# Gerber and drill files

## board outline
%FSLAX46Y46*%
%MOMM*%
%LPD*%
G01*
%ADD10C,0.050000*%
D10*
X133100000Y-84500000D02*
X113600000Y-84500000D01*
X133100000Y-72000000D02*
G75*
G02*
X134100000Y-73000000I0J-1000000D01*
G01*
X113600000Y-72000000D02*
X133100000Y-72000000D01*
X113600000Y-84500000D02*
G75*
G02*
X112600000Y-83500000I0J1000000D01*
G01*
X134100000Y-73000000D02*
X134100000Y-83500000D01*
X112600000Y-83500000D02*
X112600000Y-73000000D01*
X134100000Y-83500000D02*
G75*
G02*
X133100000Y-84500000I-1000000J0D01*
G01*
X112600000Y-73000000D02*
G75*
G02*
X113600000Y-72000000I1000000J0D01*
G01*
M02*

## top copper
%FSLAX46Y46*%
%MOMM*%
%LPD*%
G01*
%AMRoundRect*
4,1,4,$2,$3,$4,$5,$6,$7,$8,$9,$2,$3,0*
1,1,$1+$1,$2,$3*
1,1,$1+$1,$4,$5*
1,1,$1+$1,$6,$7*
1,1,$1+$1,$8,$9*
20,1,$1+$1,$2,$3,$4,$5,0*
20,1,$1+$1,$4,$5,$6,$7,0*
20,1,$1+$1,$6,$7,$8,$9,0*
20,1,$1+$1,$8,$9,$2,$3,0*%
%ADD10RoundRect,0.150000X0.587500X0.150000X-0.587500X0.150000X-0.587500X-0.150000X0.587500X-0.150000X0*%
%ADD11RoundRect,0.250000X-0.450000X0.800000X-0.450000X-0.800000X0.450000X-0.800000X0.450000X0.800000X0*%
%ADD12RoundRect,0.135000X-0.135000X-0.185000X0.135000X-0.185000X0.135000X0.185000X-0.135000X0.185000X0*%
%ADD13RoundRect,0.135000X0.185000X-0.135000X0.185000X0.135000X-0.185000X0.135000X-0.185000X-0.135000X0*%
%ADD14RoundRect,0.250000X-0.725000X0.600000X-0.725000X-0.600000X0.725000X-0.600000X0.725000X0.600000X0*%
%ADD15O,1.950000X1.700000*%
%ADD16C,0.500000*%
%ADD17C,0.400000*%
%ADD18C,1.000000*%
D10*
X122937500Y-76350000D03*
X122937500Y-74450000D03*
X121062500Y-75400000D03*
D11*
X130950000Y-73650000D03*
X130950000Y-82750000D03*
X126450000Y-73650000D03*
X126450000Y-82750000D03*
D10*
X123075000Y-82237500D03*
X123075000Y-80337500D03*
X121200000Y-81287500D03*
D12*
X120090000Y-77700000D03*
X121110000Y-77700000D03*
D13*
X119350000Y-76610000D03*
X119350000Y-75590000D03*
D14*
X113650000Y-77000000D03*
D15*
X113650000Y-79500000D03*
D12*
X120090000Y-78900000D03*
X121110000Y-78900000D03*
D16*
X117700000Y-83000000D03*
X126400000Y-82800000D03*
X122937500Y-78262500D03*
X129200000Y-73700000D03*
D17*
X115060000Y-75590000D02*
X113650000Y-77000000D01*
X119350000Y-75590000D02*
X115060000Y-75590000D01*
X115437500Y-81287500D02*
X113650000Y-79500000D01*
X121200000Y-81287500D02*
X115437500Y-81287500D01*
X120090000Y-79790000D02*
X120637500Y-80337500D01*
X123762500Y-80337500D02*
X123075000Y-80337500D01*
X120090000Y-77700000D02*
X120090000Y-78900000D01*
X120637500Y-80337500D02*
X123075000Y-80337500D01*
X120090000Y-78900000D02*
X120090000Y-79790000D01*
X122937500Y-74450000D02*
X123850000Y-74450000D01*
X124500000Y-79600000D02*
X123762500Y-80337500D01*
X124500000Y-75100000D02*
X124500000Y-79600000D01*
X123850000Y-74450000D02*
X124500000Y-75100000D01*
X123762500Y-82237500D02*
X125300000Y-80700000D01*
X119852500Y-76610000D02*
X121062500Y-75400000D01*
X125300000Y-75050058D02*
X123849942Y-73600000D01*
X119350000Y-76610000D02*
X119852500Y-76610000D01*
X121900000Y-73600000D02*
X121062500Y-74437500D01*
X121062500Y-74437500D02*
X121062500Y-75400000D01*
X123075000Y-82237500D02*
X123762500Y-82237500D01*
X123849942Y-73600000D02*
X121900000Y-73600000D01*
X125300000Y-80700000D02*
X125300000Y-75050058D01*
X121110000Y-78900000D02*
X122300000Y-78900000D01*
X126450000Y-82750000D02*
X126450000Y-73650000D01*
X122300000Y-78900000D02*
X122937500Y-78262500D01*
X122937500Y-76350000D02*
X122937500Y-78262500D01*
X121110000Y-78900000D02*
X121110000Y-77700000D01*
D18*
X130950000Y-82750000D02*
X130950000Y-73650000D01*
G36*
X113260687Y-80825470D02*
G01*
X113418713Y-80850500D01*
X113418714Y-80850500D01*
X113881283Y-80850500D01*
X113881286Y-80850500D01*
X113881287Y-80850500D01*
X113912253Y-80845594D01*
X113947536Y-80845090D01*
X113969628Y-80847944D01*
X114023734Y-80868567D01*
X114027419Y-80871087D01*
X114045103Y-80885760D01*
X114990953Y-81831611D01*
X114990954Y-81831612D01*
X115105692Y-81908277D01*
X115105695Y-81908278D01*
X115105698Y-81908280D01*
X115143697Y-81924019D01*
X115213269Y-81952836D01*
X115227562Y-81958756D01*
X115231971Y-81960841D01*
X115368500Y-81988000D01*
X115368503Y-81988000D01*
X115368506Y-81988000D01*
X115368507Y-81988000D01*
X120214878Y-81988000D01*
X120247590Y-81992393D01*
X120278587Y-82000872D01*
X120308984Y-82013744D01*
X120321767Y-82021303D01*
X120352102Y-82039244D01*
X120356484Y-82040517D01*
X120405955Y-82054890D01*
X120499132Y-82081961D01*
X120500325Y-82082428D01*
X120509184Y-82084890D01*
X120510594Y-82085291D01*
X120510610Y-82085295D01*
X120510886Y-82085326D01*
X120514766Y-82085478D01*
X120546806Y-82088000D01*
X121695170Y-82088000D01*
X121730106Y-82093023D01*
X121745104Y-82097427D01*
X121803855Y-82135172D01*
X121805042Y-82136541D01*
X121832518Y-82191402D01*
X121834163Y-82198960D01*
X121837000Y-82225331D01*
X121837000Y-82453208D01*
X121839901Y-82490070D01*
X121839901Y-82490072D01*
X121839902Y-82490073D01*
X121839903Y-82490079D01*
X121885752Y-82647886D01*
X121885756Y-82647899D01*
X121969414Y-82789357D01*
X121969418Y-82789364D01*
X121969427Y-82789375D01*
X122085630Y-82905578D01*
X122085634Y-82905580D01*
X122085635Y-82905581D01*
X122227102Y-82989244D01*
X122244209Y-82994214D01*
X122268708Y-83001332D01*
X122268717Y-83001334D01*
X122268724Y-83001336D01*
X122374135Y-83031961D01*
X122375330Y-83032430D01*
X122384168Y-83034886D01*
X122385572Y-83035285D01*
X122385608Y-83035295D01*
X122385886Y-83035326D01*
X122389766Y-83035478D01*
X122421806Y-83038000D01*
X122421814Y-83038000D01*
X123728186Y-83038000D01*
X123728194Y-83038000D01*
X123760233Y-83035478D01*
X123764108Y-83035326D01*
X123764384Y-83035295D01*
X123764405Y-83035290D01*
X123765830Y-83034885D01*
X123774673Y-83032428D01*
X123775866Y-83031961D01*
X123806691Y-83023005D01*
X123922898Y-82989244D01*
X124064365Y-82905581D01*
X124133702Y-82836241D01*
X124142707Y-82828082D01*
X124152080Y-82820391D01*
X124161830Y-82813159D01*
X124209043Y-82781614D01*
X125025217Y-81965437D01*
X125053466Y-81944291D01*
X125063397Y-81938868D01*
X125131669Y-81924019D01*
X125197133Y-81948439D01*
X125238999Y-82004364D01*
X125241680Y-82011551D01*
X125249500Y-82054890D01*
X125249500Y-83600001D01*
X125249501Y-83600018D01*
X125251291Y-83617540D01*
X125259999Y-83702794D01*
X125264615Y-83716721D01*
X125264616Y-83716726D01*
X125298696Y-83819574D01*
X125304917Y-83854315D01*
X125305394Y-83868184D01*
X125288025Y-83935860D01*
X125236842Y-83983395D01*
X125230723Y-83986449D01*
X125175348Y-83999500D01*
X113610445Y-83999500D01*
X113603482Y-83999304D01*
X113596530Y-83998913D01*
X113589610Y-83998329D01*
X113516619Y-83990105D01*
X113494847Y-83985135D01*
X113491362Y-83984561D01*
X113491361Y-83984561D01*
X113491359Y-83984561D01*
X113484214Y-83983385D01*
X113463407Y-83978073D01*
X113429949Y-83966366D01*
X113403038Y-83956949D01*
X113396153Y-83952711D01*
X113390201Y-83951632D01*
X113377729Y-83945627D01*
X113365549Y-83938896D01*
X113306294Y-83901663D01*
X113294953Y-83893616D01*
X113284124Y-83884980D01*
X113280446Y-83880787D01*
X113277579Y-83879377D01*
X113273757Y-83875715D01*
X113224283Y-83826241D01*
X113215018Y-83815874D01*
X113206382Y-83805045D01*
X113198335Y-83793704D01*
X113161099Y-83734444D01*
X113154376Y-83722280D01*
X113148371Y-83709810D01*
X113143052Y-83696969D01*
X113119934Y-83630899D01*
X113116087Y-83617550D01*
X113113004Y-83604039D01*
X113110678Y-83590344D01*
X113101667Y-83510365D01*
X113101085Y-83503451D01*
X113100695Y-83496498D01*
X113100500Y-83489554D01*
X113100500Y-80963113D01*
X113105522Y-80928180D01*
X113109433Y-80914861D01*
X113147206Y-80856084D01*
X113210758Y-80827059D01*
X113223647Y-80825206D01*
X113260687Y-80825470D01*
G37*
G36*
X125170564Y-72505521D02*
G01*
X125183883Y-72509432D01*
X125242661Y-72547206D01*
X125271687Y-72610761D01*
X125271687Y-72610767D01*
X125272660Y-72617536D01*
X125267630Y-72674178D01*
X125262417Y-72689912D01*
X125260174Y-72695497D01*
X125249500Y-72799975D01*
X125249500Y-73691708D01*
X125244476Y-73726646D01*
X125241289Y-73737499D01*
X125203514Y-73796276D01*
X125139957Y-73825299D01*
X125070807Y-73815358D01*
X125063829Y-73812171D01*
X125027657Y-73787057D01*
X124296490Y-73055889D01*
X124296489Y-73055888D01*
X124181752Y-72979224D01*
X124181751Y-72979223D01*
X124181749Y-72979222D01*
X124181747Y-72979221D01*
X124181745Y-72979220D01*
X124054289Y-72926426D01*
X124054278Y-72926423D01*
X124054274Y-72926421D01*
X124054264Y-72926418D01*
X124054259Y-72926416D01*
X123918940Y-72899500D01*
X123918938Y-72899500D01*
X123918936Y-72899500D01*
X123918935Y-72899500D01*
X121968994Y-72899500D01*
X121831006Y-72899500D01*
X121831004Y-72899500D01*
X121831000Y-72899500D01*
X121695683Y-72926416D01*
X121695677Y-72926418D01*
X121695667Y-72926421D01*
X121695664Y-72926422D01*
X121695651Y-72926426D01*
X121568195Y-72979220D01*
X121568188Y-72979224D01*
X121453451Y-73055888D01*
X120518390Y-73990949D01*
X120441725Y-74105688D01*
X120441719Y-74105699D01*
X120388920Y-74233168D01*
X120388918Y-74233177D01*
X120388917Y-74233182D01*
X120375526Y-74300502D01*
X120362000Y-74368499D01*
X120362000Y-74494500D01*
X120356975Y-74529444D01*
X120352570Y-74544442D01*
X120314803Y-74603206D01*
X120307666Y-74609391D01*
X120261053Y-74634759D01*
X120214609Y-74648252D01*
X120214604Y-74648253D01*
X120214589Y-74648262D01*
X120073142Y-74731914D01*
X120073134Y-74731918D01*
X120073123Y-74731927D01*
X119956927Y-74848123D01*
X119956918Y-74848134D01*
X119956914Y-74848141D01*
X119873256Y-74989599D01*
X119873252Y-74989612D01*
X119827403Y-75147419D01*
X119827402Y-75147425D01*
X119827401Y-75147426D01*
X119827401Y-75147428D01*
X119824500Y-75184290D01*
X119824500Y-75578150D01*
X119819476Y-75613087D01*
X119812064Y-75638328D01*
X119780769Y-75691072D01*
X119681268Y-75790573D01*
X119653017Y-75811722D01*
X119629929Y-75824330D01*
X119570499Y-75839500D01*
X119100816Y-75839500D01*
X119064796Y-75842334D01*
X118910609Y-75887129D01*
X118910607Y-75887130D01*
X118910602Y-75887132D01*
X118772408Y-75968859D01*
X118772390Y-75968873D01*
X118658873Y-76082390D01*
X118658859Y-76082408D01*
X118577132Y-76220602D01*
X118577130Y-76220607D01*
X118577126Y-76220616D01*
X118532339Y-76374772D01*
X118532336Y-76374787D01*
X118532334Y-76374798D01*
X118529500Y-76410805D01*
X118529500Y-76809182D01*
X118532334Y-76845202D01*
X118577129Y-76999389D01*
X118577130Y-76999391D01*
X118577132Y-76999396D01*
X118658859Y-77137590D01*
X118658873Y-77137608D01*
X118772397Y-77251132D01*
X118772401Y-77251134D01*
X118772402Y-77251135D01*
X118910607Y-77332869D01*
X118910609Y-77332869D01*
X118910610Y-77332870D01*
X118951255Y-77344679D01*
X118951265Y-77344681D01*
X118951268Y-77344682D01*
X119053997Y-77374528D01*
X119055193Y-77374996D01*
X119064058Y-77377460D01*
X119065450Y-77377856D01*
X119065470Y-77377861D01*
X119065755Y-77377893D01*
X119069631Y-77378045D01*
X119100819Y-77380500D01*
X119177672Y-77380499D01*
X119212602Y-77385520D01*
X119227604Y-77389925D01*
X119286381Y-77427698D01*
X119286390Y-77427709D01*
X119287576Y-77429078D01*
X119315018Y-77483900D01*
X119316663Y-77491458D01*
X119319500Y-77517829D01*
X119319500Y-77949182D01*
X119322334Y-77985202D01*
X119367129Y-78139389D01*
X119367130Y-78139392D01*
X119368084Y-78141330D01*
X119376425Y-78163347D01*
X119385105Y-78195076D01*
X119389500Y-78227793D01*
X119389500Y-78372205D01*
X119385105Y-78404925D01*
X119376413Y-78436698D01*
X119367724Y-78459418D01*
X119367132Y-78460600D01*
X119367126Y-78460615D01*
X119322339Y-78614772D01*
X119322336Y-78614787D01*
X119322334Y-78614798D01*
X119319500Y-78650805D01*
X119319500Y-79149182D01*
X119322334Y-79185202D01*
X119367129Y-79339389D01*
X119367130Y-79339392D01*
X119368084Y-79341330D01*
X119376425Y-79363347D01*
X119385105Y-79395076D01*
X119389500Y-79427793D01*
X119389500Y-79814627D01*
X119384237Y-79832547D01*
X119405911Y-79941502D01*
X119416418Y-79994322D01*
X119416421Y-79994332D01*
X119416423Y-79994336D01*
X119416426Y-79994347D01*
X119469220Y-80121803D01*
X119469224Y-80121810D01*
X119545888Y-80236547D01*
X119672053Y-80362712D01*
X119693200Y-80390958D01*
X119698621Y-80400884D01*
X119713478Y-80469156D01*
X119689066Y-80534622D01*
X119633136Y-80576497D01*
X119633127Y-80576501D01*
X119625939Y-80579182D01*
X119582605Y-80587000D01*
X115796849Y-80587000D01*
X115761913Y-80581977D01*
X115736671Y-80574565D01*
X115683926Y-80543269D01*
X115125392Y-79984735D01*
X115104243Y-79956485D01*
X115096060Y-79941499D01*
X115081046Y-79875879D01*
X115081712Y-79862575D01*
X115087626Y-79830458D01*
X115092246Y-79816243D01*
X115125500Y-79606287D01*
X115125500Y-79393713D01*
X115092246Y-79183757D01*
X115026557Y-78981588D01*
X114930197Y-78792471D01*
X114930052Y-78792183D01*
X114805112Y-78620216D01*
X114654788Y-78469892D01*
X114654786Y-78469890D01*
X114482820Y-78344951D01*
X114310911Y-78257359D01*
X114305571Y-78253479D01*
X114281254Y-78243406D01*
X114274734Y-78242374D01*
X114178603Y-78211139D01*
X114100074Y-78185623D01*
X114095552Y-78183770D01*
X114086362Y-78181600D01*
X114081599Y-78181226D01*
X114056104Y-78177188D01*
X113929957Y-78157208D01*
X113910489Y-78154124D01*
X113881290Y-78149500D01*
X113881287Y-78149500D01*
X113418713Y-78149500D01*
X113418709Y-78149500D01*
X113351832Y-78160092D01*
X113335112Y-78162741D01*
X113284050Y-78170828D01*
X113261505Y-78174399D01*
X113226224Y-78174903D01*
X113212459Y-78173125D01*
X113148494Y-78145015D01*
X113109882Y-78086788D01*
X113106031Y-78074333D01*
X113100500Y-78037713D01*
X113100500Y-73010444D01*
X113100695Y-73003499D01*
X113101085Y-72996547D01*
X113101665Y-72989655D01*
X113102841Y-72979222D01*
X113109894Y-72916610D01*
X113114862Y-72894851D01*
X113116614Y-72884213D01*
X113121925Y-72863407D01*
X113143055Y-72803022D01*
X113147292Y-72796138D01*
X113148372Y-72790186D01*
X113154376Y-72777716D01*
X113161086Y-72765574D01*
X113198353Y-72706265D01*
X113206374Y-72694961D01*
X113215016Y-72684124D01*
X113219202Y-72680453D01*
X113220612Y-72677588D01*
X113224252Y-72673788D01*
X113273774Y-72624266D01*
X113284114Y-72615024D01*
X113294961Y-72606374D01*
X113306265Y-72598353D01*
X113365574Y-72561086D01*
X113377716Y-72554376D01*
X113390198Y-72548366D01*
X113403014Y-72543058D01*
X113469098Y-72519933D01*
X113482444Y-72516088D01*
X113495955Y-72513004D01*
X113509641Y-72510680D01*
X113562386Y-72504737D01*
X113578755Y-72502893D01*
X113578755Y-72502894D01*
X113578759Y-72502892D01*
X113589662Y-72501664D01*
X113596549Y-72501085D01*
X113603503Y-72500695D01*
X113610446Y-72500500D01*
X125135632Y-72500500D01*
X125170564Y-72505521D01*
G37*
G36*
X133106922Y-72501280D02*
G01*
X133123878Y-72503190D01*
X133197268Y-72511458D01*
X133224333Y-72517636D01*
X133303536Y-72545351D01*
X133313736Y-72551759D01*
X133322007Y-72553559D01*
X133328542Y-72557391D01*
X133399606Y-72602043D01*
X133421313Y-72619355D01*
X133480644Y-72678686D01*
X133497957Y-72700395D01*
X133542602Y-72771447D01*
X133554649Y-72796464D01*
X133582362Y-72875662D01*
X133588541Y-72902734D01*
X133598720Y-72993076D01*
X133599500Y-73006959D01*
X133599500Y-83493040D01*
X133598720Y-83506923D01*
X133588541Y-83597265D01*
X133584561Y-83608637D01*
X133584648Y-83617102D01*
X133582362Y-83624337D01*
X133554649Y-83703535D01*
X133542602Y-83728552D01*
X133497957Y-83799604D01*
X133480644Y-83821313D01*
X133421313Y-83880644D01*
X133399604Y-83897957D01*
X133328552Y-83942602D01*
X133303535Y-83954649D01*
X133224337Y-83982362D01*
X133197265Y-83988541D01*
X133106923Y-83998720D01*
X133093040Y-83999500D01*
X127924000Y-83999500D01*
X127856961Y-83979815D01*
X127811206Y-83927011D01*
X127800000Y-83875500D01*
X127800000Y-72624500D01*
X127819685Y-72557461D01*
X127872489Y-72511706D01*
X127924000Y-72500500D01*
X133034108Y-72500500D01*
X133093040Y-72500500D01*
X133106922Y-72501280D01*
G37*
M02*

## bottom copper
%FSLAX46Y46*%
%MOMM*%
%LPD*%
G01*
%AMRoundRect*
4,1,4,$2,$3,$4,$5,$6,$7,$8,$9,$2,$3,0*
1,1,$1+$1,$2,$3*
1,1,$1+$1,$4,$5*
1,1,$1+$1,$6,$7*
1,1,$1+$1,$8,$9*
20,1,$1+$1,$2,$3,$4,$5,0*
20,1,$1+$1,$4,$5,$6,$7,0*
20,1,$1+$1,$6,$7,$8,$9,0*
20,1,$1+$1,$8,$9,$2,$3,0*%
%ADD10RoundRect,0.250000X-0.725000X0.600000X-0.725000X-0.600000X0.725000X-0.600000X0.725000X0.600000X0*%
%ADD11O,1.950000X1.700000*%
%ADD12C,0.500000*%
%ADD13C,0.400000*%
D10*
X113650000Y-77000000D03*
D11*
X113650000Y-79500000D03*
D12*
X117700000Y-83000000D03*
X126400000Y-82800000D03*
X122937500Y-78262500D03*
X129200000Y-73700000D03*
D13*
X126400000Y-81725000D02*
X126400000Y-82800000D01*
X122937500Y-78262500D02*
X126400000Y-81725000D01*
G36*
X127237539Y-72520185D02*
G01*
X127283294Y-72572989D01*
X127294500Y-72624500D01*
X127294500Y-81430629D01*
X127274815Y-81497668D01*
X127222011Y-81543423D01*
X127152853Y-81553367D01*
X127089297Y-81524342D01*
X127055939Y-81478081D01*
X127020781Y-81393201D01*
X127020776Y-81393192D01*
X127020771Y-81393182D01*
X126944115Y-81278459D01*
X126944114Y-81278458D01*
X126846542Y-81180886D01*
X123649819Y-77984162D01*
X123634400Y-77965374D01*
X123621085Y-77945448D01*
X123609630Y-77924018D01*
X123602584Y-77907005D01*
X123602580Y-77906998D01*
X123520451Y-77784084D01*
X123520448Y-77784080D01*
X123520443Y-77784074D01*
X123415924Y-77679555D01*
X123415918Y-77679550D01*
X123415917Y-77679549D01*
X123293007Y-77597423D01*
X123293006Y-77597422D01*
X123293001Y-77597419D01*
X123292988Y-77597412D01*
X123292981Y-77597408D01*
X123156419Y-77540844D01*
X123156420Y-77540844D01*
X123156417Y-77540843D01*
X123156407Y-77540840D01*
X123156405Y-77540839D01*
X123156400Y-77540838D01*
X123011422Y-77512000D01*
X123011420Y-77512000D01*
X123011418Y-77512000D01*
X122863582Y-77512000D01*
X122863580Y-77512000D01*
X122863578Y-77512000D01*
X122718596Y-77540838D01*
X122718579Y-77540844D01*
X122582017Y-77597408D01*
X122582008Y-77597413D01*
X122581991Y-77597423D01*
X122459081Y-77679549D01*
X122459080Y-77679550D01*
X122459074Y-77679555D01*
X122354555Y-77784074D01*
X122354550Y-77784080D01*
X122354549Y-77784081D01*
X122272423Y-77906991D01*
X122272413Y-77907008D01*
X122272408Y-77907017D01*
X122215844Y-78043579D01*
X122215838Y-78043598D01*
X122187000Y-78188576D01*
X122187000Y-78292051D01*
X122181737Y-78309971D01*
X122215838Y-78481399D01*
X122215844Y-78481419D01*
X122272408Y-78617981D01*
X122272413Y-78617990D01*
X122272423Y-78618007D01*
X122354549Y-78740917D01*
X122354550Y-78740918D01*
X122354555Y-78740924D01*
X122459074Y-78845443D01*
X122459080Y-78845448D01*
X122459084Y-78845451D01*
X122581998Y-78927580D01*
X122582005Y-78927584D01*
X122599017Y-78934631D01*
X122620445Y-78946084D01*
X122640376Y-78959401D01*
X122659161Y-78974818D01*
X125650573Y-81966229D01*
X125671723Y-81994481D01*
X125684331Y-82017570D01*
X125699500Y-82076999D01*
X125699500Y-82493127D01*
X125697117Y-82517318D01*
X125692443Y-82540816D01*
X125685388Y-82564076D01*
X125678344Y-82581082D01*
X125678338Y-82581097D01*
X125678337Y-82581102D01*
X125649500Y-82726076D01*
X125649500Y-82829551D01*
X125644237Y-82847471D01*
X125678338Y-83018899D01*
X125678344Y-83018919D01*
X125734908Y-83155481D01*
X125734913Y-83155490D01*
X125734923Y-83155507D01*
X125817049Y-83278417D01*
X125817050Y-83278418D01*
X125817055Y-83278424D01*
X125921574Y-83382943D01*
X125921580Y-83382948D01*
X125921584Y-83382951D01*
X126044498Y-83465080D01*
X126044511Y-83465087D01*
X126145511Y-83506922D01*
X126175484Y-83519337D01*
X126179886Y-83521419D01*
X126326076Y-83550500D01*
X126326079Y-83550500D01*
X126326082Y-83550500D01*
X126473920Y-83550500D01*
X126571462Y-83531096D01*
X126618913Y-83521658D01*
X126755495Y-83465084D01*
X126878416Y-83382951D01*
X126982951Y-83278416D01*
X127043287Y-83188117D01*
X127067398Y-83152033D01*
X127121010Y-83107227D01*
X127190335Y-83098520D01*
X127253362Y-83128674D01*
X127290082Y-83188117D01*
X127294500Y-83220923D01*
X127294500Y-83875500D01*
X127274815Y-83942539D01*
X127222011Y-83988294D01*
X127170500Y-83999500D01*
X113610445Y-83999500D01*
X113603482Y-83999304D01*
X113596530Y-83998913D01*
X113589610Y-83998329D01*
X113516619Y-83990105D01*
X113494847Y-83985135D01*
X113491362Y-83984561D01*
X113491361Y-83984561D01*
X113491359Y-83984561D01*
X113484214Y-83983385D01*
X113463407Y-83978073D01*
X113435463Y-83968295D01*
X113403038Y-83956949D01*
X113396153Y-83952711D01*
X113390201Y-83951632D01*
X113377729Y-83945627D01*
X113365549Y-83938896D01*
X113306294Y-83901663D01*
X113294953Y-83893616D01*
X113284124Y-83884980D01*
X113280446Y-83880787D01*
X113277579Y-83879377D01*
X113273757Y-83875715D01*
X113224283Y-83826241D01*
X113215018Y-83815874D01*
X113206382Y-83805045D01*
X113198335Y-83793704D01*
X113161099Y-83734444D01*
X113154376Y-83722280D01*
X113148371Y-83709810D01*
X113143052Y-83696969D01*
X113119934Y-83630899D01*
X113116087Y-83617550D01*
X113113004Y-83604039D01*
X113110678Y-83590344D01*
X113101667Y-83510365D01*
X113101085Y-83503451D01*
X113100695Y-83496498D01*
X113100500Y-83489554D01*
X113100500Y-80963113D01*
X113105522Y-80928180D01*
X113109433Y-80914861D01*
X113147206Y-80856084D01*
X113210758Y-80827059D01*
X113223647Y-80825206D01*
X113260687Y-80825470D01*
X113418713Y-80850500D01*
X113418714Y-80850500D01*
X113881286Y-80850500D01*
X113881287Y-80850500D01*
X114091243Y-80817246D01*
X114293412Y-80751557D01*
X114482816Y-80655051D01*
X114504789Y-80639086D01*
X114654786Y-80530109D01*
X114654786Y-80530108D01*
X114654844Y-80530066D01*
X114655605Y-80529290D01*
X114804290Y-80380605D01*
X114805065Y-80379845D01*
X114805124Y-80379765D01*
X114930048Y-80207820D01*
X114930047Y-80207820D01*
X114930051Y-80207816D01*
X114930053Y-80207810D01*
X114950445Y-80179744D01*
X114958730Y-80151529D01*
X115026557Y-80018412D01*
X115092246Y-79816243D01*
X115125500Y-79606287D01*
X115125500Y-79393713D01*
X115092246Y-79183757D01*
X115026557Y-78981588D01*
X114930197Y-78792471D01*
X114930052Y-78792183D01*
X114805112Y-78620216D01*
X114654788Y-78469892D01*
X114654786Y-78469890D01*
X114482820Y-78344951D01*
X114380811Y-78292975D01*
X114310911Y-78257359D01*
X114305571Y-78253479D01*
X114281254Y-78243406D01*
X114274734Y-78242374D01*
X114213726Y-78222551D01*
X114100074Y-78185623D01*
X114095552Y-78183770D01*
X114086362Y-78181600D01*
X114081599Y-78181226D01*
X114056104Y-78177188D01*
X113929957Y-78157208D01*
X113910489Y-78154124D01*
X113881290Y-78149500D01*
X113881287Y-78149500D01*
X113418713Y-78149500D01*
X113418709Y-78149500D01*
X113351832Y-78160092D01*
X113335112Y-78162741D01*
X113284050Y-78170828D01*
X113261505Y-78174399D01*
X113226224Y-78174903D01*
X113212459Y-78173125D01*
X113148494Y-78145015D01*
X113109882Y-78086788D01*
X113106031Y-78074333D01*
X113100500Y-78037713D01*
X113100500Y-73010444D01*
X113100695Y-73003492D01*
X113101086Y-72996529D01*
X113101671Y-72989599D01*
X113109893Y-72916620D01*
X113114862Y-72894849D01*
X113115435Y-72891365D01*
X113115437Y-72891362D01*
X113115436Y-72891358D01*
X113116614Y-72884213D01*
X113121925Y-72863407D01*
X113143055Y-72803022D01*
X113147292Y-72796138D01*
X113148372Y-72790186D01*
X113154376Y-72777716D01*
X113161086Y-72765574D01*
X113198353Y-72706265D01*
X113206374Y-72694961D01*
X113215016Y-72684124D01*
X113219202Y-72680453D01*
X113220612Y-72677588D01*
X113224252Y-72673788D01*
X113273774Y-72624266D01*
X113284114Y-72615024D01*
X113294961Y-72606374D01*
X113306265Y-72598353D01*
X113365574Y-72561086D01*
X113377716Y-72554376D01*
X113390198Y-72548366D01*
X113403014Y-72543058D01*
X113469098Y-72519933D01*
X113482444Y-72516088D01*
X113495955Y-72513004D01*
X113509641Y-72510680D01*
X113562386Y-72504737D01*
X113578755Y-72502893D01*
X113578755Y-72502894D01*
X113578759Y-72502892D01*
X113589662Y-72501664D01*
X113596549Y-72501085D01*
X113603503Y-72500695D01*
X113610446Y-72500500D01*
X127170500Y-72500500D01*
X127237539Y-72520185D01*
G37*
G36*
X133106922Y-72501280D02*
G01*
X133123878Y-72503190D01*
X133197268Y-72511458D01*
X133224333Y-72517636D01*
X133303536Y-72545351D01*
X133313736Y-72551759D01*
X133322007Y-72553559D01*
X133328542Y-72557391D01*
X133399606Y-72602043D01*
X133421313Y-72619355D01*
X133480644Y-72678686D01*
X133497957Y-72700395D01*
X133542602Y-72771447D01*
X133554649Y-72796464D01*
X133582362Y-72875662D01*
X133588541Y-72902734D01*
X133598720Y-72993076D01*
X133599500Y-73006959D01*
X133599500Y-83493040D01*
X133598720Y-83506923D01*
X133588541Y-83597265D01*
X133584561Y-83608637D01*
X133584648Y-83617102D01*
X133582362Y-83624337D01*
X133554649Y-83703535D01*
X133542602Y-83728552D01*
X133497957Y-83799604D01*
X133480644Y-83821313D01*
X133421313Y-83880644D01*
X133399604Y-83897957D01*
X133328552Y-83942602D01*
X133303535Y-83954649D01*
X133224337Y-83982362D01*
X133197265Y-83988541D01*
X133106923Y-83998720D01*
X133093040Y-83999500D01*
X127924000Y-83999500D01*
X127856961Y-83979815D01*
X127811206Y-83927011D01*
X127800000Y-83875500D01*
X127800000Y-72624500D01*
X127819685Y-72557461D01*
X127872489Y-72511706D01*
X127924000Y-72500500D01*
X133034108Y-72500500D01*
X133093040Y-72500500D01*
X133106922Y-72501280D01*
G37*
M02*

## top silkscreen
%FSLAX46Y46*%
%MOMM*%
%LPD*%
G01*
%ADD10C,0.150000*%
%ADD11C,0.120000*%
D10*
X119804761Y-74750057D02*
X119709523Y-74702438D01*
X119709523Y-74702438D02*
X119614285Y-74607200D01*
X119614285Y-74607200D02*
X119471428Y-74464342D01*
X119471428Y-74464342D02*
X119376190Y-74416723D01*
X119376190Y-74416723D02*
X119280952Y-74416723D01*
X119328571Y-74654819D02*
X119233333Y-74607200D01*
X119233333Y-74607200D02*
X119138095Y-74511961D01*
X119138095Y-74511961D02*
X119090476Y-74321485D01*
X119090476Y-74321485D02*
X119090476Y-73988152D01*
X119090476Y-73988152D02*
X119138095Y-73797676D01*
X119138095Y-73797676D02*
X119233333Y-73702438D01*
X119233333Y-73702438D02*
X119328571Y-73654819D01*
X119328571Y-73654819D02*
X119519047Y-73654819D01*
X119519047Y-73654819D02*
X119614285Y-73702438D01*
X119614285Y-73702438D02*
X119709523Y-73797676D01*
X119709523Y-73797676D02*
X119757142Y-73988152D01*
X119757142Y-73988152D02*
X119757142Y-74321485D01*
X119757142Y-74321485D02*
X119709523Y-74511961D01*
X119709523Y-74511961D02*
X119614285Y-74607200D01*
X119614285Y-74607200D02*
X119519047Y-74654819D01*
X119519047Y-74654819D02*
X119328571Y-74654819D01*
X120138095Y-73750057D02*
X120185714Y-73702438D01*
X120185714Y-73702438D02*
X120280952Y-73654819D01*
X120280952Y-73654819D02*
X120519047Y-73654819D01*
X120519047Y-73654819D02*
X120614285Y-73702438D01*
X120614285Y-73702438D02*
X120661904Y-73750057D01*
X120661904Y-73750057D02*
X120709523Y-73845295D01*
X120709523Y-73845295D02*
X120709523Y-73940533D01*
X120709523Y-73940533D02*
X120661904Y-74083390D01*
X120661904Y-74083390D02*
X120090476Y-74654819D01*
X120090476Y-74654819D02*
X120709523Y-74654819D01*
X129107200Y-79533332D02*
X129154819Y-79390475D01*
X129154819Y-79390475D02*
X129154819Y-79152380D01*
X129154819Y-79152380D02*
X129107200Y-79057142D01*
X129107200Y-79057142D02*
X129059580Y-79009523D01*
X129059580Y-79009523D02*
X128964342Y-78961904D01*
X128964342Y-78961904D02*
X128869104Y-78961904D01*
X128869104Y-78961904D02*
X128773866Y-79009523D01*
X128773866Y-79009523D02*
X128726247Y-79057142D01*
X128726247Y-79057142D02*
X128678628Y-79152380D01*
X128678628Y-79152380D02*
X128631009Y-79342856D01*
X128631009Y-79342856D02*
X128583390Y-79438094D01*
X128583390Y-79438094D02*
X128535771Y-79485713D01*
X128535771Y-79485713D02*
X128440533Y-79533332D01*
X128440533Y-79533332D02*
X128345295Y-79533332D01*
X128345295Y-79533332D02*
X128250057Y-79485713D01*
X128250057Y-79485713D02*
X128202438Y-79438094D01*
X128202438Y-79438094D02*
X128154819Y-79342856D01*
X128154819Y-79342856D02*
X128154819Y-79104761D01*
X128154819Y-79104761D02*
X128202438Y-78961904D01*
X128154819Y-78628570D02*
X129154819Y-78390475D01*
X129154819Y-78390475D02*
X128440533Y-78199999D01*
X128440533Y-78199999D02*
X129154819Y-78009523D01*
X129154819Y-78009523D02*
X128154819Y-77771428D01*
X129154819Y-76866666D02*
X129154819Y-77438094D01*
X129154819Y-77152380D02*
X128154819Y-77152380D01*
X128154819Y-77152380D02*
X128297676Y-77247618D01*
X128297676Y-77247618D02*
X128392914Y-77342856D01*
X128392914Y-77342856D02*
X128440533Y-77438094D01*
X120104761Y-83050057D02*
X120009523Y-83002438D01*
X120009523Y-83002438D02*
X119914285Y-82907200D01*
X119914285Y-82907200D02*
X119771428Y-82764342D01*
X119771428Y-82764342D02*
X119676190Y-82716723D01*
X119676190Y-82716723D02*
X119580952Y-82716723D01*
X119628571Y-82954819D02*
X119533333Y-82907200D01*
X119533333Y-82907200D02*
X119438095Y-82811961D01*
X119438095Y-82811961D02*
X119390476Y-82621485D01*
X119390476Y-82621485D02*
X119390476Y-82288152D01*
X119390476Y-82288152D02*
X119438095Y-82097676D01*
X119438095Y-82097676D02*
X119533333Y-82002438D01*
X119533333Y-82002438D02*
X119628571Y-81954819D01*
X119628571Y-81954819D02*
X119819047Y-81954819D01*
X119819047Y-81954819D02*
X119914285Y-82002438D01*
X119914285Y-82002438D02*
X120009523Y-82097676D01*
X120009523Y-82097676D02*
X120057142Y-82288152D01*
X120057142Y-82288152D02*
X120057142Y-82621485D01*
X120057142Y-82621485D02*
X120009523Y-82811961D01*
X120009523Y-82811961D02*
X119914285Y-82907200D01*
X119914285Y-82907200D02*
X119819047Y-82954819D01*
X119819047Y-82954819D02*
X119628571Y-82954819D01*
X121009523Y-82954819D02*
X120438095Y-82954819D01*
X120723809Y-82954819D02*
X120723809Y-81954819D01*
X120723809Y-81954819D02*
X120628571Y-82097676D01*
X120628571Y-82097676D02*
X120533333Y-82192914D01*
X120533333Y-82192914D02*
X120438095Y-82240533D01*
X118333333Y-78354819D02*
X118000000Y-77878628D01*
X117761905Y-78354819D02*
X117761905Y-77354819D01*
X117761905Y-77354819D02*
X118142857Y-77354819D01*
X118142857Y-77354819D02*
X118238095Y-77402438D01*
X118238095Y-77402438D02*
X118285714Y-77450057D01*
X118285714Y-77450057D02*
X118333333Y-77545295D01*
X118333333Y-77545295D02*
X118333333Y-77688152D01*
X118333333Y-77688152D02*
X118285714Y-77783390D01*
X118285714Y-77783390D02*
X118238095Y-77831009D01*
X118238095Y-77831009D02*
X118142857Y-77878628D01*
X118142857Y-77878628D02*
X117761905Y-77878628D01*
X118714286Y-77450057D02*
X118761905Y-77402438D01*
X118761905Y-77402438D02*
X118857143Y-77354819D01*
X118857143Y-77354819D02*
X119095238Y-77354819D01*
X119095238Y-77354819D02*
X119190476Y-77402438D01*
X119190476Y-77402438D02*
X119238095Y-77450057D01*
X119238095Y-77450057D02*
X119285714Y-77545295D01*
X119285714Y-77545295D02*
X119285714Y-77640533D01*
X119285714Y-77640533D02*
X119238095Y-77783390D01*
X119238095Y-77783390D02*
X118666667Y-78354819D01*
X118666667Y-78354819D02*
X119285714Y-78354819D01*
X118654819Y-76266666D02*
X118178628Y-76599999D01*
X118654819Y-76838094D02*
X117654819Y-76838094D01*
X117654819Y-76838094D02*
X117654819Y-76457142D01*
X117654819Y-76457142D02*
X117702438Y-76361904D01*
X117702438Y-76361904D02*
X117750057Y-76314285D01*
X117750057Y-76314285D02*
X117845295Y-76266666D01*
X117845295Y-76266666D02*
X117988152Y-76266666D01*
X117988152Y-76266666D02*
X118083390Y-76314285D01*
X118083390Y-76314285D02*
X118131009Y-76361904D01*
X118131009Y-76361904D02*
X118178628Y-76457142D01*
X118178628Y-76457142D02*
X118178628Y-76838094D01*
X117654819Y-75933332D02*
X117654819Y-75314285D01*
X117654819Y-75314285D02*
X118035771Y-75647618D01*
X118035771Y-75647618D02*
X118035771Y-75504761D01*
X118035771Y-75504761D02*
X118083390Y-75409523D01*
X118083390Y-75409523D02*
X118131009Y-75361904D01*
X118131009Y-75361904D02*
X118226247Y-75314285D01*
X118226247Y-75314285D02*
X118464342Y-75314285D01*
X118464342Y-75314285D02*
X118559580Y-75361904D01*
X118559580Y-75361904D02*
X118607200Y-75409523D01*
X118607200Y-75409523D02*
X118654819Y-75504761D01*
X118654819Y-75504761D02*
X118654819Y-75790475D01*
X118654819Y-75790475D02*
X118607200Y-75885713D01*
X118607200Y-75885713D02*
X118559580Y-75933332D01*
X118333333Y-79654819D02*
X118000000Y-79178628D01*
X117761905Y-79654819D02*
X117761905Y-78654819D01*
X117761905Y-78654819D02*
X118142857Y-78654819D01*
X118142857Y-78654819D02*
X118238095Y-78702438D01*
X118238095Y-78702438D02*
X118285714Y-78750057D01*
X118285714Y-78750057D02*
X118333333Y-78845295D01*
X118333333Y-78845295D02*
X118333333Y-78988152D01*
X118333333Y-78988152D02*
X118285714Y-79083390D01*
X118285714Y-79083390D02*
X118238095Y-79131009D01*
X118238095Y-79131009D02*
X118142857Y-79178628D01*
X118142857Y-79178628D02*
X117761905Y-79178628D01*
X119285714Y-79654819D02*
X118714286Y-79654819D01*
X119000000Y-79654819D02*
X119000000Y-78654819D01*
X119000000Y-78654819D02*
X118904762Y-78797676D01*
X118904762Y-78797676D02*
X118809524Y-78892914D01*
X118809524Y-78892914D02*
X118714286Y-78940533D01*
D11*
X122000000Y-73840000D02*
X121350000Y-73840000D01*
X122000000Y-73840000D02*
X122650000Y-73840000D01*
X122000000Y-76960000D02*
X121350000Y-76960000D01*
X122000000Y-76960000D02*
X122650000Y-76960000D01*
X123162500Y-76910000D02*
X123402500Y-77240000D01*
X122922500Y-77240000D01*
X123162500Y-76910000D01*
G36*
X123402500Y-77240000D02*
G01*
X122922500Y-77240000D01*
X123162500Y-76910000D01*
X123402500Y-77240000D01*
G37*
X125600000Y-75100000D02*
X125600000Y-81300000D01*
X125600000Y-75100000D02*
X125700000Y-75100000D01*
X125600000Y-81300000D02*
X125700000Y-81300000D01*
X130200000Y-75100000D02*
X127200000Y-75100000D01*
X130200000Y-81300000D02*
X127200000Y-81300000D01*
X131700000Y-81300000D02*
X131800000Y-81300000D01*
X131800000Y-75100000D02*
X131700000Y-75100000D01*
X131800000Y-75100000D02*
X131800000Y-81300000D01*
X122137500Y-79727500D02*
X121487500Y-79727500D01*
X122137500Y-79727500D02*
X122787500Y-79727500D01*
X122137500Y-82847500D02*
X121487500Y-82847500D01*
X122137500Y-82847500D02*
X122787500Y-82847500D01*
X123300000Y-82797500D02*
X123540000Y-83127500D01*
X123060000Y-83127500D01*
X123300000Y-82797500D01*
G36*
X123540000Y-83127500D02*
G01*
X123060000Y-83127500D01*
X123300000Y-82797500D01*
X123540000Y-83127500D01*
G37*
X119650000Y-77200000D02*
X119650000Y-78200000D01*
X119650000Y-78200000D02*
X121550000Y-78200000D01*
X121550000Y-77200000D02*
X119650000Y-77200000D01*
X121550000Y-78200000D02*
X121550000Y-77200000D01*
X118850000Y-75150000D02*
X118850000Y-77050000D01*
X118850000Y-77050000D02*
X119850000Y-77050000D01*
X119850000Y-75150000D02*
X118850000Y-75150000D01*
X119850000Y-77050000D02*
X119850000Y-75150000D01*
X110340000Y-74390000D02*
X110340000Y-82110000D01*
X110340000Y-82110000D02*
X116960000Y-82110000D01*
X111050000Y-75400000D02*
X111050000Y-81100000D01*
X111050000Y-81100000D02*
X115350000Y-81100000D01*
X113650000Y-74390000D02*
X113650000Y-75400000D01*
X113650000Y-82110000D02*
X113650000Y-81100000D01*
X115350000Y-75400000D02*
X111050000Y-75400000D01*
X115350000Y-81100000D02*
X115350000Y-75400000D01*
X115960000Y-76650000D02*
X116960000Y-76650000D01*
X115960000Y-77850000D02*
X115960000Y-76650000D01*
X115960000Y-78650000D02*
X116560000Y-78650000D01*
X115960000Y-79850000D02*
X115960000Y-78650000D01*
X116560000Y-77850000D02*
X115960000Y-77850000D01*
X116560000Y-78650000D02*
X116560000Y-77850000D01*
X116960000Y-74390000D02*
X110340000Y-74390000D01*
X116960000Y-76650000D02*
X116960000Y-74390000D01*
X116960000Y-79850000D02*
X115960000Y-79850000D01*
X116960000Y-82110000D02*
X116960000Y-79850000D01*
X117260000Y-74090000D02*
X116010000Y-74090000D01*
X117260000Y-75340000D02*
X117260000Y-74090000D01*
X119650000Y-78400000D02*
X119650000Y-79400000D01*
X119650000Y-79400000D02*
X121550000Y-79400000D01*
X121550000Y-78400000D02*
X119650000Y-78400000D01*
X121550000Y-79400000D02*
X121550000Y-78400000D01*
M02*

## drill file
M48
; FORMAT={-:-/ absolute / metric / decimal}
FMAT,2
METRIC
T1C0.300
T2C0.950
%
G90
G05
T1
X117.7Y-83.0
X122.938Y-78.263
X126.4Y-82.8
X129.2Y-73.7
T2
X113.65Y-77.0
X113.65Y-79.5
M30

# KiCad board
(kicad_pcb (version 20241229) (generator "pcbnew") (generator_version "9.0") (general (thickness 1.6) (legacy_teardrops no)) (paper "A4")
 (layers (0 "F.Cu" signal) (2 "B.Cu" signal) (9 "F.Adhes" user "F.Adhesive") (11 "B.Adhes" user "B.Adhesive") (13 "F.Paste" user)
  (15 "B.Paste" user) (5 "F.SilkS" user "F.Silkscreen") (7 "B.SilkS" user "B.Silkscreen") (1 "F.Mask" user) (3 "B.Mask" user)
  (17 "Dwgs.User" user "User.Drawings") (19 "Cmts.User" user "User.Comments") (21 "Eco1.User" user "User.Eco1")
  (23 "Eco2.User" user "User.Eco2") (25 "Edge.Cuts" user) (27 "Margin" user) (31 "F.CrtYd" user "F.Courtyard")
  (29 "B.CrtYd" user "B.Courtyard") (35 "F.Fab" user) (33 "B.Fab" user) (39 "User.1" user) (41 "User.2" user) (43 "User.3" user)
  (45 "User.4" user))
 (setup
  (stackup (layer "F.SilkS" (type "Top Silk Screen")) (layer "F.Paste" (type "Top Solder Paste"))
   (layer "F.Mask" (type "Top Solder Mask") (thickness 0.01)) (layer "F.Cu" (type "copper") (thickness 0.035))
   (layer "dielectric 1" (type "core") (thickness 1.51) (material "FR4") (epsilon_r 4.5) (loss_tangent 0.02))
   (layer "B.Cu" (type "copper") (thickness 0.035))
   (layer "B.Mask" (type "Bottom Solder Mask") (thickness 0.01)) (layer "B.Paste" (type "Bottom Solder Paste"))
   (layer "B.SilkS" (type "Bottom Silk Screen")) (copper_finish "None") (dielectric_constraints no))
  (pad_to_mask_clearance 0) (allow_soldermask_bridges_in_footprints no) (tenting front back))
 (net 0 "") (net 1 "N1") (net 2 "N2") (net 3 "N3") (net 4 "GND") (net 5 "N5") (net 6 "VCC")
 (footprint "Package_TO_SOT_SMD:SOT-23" (layer "F.Cu") (at 122 75.4 180)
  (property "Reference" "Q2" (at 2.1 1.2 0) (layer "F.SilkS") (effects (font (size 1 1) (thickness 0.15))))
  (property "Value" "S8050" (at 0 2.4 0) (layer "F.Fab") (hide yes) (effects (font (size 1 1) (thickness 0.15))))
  (fp_line (start 0 1.56) (end 0.65 1.56) (stroke (width 0.12) (type solid)) (layer "F.SilkS"))
  (fp_line (start 0 1.56) (end -0.65 1.56) (stroke (width 0.12) (type solid)) (layer "F.SilkS"))
  (fp_line (start 0 -1.56) (end 0.65 -1.56) (stroke (width 0.12) (type solid)) (layer "F.SilkS"))
  (fp_line (start 0 -1.56) (end -0.65 -1.56) (stroke (width 0.12) (type solid)) (layer "F.SilkS"))
  (fp_poly (pts (xy -1.1625 -1.51) (xy -1.4025 -1.84) (xy -0.9225 -1.84)) (stroke (width 0.12) (type solid)) (fill yes) (layer "F.SilkS"))
  (pad "1" smd roundrect (at -0.9375 -0.95 180) (size 1.475 0.6) (layers "F.Cu" "F.Mask" "F.Paste") (roundrect_rratio 0.25) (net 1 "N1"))
  (pad "2" smd roundrect (at -0.9375 0.95 180) (size 1.475 0.6) (layers "F.Cu" "F.Mask" "F.Paste") (roundrect_rratio 0.25) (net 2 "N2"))
  (pad "3" smd roundrect (at 0.9375 0 180) (size 1.475 0.6) (layers "F.Cu" "F.Mask" "F.Paste") (roundrect_rratio 0.25) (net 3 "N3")))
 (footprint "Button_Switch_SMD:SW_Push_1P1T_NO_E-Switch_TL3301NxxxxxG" (layer "F.Cu") (at 128.7 78.2 -90)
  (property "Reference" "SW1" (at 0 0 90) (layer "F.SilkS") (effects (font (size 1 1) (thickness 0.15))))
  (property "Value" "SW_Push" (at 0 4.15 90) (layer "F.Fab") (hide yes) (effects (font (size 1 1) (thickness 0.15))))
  (fp_line (start -3.1 3.1) (end 3.1 3.1) (stroke (width 0.12) (type solid)) (layer "F.SilkS"))
  (fp_line (start -3.1 3.1) (end -3.1 3) (stroke (width 0.12) (type solid)) (layer "F.SilkS"))
  (fp_line (start 3.1 3.1) (end 3.1 3) (stroke (width 0.12) (type solid)) (layer "F.SilkS"))
  (fp_line (start -3.1 -1.5) (end -3.1 1.5) (stroke (width 0.12) (type solid)) (layer "F.SilkS"))
  (fp_line (start 3.1 -1.5) (end 3.1 1.5) (stroke (width 0.12) (type solid)) (layer "F.SilkS"))
  (fp_line (start 3.1 -3) (end 3.1 -3.1) (stroke (width 0.12) (type solid)) (layer "F.SilkS"))
  (fp_line (start -3.1 -3.1) (end -3.1 -3) (stroke (width 0.12) (type solid)) (layer "F.SilkS"))
  (fp_line (start -3.1 -3.1) (end 3.1 -3.1) (stroke (width 0.12) (type solid)) (layer "F.SilkS"))
  (pad "1" smd roundrect (at -4.55 -2.25 270) (size 2.1 1.4) (layers "F.Cu" "F.Mask" "F.Paste") (roundrect_rratio 0.1785714286)
   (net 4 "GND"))
  (pad "1" smd roundrect (at 4.55 -2.25 270) (size 2.1 1.4) (layers "F.Cu" "F.Mask" "F.Paste") (roundrect_rratio 0.1785714286) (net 4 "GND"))
  (pad "2" smd roundrect (at -4.55 2.25 270) (size 2.1 1.4) (layers "F.Cu" "F.Mask" "F.Paste") (roundrect_rratio 0.1785714286) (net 1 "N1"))
  (pad "2" smd roundrect (at 4.55 2.25 270) (size 2.1 1.4) (layers "F.Cu" "F.Mask" "F.Paste") (roundrect_rratio 0.1785714286) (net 1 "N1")))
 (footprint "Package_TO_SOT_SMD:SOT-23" (layer "F.Cu") (at 122.1375 81.2875 180)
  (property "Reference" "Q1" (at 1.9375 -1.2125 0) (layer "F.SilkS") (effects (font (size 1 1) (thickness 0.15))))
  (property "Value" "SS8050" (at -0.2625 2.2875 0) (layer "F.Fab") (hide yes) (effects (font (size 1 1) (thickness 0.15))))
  (fp_line (start 0 1.56) (end 0.65 1.56) (stroke (width 0.12) (type solid)) (layer "F.SilkS"))
  (fp_line (start 0 1.56) (end -0.65 1.56) (stroke (width 0.12) (type solid)) (layer "F.SilkS"))
  (fp_line (start 0 -1.56) (end 0.65 -1.56) (stroke (width 0.12) (type solid)) (layer "F.SilkS"))
  (fp_line (start 0 -1.56) (end -0.65 -1.56) (stroke (width 0.12) (type solid)) (layer "F.SilkS"))
  (fp_poly (pts (xy -1.1625 -1.51) (xy -1.4025 -1.84) (xy -0.9225 -1.84)) (stroke (width 0.12) (type solid)) (fill yes) (layer "F.SilkS"))
  (pad "1" smd roundrect (at -0.9375 -0.95 180) (size 1.475 0.6) (layers "F.Cu" "F.Mask" "F.Paste") (roundrect_rratio 0.25) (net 3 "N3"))
  (pad "2" smd roundrect (at -0.9375 0.95 180) (size 1.475 0.6) (layers "F.Cu" "F.Mask" "F.Paste") (roundrect_rratio 0.25) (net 2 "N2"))
  (pad "3" smd roundrect (at 0.9375 0 180) (size 1.475 0.6) (layers "F.Cu" "F.Mask" "F.Paste") (roundrect_rratio 0.25) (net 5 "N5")))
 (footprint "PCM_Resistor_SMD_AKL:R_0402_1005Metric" (layer "F.Cu") (at 120.6 77.7)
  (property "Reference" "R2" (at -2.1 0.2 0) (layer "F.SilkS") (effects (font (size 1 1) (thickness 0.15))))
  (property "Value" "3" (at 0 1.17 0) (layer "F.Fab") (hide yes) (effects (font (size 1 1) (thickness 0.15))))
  (fp_line (start -0.95 -0.5) (end -0.95 0.5) (stroke (width 0.12) (type solid)) (layer "F.SilkS"))
  (fp_line (start -0.95 0.5) (end 0.95 0.5) (stroke (width 0.12) (type solid)) (layer "F.SilkS"))
  (fp_line (start 0.95 -0.5) (end -0.95 -0.5) (stroke (width 0.12) (type solid)) (layer "F.SilkS"))
  (fp_line (start 0.95 0.5) (end 0.95 -0.5) (stroke (width 0.12) (type solid)) (layer "F.SilkS"))
  (pad "1" smd roundrect (at -0.51 0) (size 0.54 0.64) (layers "F.Cu" "F.Mask" "F.Paste") (roundrect_rratio 0.25) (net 2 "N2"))
  (pad "2" smd roundrect (at 0.51 0) (size 0.54 0.64) (layers "F.Cu" "F.Mask" "F.Paste") (roundrect_rratio 0.25) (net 1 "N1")))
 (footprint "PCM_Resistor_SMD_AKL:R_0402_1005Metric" (layer "F.Cu") (at 119.35 76.1 90)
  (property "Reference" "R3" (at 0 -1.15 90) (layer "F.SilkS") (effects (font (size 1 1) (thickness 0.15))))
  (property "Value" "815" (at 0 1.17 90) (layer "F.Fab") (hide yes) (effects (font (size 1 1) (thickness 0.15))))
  (fp_line (start 0.95 -0.5) (end -0.95 -0.5) (stroke (width 0.12) (type solid)) (layer "F.SilkS"))
  (fp_line (start -0.95 -0.5) (end -0.95 0.5) (stroke (width 0.12) (type solid)) (layer "F.SilkS"))
  (fp_line (start 0.95 0.5) (end 0.95 -0.5) (stroke (width 0.12) (type solid)) (layer "F.SilkS"))
  (fp_line (start -0.95 0.5) (end 0.95 0.5) (stroke (width 0.12) (type solid)) (layer "F.SilkS"))
  (pad "1" smd roundrect (at -0.51 0 90) (size 0.54 0.64) (layers "F.Cu" "F.Mask" "F.Paste") (roundrect_rratio 0.25) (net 3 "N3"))
  (pad "2" smd roundrect (at 0.51 0 90) (size 0.54 0.64) (layers "F.Cu" "F.Mask" "F.Paste") (roundrect_rratio 0.25) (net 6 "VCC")))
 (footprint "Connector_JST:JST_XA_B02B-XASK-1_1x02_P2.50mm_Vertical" (layer "F.Cu") (at 113.65 77 -90)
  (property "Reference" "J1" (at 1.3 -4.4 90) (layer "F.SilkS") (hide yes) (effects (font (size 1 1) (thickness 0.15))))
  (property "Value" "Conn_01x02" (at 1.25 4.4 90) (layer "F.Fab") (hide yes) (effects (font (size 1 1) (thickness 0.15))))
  (fp_line (start -2.61 3.31) (end 5.11 3.31) (stroke (width 0.12) (type solid)) (layer "F.SilkS"))
  (fp_line (start 5.11 3.31) (end 5.11 -3.31) (stroke (width 0.12) (type solid)) (layer "F.SilkS"))
  (fp_line (start -1.6 2.6) (end 4.1 2.6) (stroke (width 0.12) (type solid)) (layer "F.SilkS"))
  (fp_line (start 4.1 2.6) (end 4.1 -1.7) (stroke (width 0.12) (type solid)) (layer "F.SilkS"))
  (fp_line (start -2.61 0) (end -1.6 0) (stroke (width 0.12) (type solid)) (layer "F.SilkS"))
  (fp_line (start 5.11 0) (end 4.1 0) (stroke (width 0.12) (type solid)) (layer "F.SilkS"))
  (fp_line (start -1.6 -1.7) (end -1.6 2.6) (stroke (width 0.12) (type solid)) (layer "F.SilkS"))
  (fp_line (start 4.1 -1.7) (end -1.6 -1.7) (stroke (width 0.12) (type solid)) (layer "F.SilkS"))
  (fp_line (start -0.35 -2.31) (end -0.35 -3.31) (stroke (width 0.12) (type solid)) (layer "F.SilkS"))
  (fp_line (start 0.85 -2.31) (end -0.35 -2.31) (stroke (width 0.12) (type solid)) (layer "F.SilkS"))
  (fp_line (start 1.65 -2.31) (end 1.65 -2.91) (stroke (width 0.12) (type solid)) (layer "F.SilkS"))
  (fp_line (start 2.85 -2.31) (end 1.65 -2.31) (stroke (width 0.12) (type solid)) (layer "F.SilkS"))
  (fp_line (start 0.85 -2.91) (end 0.85 -2.31) (stroke (width 0.12) (type solid)) (layer "F.SilkS"))
  (fp_line (start 1.65 -2.91) (end 0.85 -2.91) (stroke (width 0.12) (type solid)) (layer "F.SilkS"))
  (fp_line (start -2.61 -3.31) (end -2.61 3.31) (stroke (width 0.12) (type solid)) (layer "F.SilkS"))
  (fp_line (start -0.35 -3.31) (end -2.61 -3.31) (stroke (width 0.12) (type solid)) (layer "F.SilkS"))
  (fp_line (start 2.85 -3.31) (end 2.85 -2.31) (stroke (width 0.12) (type solid)) (layer "F.SilkS"))
  (fp_line (start 5.11 -3.31) (end 2.85 -3.31) (stroke (width 0.12) (type solid)) (layer "F.SilkS"))
  (fp_line (start -2.91 -3.61) (end -2.91 -2.36) (stroke (width 0.12) (type solid)) (layer "F.SilkS"))
  (fp_line (start -1.66 -3.61) (end -2.91 -3.61) (stroke (width 0.12) (type solid)) (layer "F.SilkS"))
  (pad "1" thru_hole roundrect (at 0 0 270) (size 1.7 1.95) (drill 0.95) (layers "*.Cu" "*.Mask") (remove_unused_layers no)
   (roundrect_rratio 0.147059) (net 6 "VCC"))
  (pad "2" thru_hole oval (at 2.5 0 270) (size 1.7 1.95) (drill 0.95) (layers "*.Cu" "*.Mask") (remove_unused_layers no) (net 5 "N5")))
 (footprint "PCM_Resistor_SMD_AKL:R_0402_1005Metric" (layer "F.Cu") (at 120.6 78.9)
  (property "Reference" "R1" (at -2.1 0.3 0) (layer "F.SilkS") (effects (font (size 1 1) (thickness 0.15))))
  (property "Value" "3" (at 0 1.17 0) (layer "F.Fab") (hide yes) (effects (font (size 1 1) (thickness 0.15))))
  (fp_line (start -0.95 -0.5) (end -0.95 0.5) (stroke (width 0.12) (type solid)) (layer "F.SilkS"))
  (fp_line (start -0.95 0.5) (end 0.95 0.5) (stroke (width 0.12) (type solid)) (layer "F.SilkS"))
  (fp_line (start 0.95 -0.5) (end -0.95 -0.5) (stroke (width 0.12) (type solid)) (layer "F.SilkS"))
  (fp_line (start 0.95 0.5) (end 0.95 -0.5) (stroke (width 0.12) (type solid)) (layer "F.SilkS"))
  (pad "1" smd roundrect (at -0.51 0) (size 0.54 0.64) (layers "F.Cu" "F.Mask" "F.Paste") (roundrect_rratio 0.25) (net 2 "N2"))
  (pad "2" smd roundrect (at 0.51 0) (size 0.54 0.64) (layers "F.Cu" "F.Mask" "F.Paste") (roundrect_rratio 0.25) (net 1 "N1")))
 (gr_line (start 133.1 84.5) (end 113.6 84.5) (stroke (width 0.05) (type default)) (layer "Edge.Cuts"))
 (gr_arc (start 133.1 72) (mid 133.807107 72.292893) (end 134.1 73) (stroke (width 0.05) (type default)) (layer "Edge.Cuts"))
 (gr_line (start 113.6 72) (end 133.1 72) (stroke (width 0.05) (type default)) (layer "Edge.Cuts"))
 (gr_arc (start 113.6 84.5) (mid 112.892893 84.207107) (end 112.6 83.5) (stroke (width 0.05) (type default)) (layer "Edge.Cuts"))
 (gr_line (start 134.1 73) (end 134.1 83.5) (stroke (width 0.05) (type default)) (layer "Edge.Cuts"))
 (gr_line (start 112.6 83.5) (end 112.6 73) (stroke (width 0.05) (type default)) (layer "Edge.Cuts"))
 (gr_arc (start 134.1 83.5) (mid 133.807107 84.207107) (end 133.1 84.5) (stroke (width 0.05) (type default)) (layer "Edge.Cuts"))
 (gr_arc (start 112.6 73) (mid 112.892893 72.292893) (end 113.6 72) (stroke (width 0.05) (type default)) (layer "Edge.Cuts"))
 (segment (start 115.06 75.59) (end 113.65 77) (width 0.4) (layer "F.Cu") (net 6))
 (segment (start 119.35 75.59) (end 115.06 75.59) (width 0.4) (layer "F.Cu") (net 6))
 (via (at 117.7 83) (size 0.5) (drill 0.3) (layers "F.Cu" "B.Cu") (free yes) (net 6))
 (segment (start 115.4375 81.2875) (end 113.65 79.5) (width 0.4) (layer "F.Cu") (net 5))
 (segment (start 121.2 81.2875) (end 115.4375 81.2875) (width 0.4) (layer "F.Cu") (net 5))
 (segment (start 120.09 79.79) (end 120.6375 80.3375) (width 0.4) (layer "F.Cu") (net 2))
 (segment (start 123.7625 80.3375) (end 123.075 80.3375) (width 0.4) (layer "F.Cu") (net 2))
 (segment (start 120.09 77.7) (end 120.09 78.9) (width 0.4) (layer "F.Cu") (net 2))
 (segment (start 120.6375 80.3375) (end 123.075 80.3375) (width 0.4) (layer "F.Cu") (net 2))
 (segment (start 120.09 78.9) (end 120.09 79.79) (width 0.4) (layer "F.Cu") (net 2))
 (segment (start 122.9375 74.45) (end 123.85 74.45) (width 0.4) (layer "F.Cu") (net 2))
 (segment (start 124.5 79.6) (end 123.7625 80.3375) (width 0.4) (layer "F.Cu") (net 2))
 (segment (start 124.5 75.1) (end 124.5 79.6) (width 0.4) (layer "F.Cu") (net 2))
 (segment (start 123.85 74.45) (end 124.5 75.1) (width 0.4) (layer "F.Cu") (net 2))
 (segment (start 123.7625 82.2375) (end 125.3 80.7) (width 0.4) (layer "F.Cu") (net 3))
 (segment (start 119.8525 76.61) (end 121.0625 75.4) (width 0.4) (layer "F.Cu") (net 3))
 (segment (start 125.3 75.050058) (end 123.849942 73.6) (width 0.4) (layer "F.Cu") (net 3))
 (segment (start 119.35 76.61) (end 119.8525 76.61) (width 0.4) (layer "F.Cu") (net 3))
 (segment (start 121.9 73.6) (end 121.0625 74.4375) (width 0.4) (layer "F.Cu") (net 3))
 (segment (start 121.0625 74.4375) (end 121.0625 75.4) (width 0.4) (layer "F.Cu") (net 3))
 (segment (start 123.075 82.2375) (end 123.7625 82.2375) (width 0.4) (layer "F.Cu") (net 3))
 (segment (start 123.849942 73.6) (end 121.9 73.6) (width 0.4) (layer "F.Cu") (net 3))
 (segment (start 125.3 80.7) (end 125.3 75.050058) (width 0.4) (layer "F.Cu") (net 3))
 (segment (start 121.11 78.9) (end 122.3 78.9) (width 0.4) (layer "F.Cu") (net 1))
 (segment (start 126.45 82.75) (end 126.45 73.65) (width 0.4) (layer "F.Cu") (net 1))
 (segment (start 122.3 78.9) (end 122.9375 78.2625) (width 0.4) (layer "F.Cu") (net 1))
 (segment (start 122.9375 76.35) (end 122.9375 78.2625) (width 0.4) (layer "F.Cu") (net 1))
 (segment (start 121.11 78.9) (end 121.11 77.7) (width 0.4) (layer "F.Cu") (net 1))
 (via (at 126.4 82.8) (size 0.5) (drill 0.3) (layers "F.Cu" "B.Cu") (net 1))
 (via (at 122.9375 78.2625) (size 0.5) (drill 0.3) (layers "F.Cu" "B.Cu") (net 1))
 (segment (start 126.4 81.725) (end 126.4 82.8) (width 0.4) (layer "B.Cu") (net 1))
 (segment (start 122.9375 78.2625) (end 126.4 81.725) (width 0.4) (layer "B.Cu") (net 1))
 (segment (start 130.95 82.75) (end 130.95 73.65) (width 1) (layer "F.Cu") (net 4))
 (via (at 129.2 73.7) (size 0.5) (drill 0.3) (layers "F.Cu" "B.Cu") (free yes) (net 4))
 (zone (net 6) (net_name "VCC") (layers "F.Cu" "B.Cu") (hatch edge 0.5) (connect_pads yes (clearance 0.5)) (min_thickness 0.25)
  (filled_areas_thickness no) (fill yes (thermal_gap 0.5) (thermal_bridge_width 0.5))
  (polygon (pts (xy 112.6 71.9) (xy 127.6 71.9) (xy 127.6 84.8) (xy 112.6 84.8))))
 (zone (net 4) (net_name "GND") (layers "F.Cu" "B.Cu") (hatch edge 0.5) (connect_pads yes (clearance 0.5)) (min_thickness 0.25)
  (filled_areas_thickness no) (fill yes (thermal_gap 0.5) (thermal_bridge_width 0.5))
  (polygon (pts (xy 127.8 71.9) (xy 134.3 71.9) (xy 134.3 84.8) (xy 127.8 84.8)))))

